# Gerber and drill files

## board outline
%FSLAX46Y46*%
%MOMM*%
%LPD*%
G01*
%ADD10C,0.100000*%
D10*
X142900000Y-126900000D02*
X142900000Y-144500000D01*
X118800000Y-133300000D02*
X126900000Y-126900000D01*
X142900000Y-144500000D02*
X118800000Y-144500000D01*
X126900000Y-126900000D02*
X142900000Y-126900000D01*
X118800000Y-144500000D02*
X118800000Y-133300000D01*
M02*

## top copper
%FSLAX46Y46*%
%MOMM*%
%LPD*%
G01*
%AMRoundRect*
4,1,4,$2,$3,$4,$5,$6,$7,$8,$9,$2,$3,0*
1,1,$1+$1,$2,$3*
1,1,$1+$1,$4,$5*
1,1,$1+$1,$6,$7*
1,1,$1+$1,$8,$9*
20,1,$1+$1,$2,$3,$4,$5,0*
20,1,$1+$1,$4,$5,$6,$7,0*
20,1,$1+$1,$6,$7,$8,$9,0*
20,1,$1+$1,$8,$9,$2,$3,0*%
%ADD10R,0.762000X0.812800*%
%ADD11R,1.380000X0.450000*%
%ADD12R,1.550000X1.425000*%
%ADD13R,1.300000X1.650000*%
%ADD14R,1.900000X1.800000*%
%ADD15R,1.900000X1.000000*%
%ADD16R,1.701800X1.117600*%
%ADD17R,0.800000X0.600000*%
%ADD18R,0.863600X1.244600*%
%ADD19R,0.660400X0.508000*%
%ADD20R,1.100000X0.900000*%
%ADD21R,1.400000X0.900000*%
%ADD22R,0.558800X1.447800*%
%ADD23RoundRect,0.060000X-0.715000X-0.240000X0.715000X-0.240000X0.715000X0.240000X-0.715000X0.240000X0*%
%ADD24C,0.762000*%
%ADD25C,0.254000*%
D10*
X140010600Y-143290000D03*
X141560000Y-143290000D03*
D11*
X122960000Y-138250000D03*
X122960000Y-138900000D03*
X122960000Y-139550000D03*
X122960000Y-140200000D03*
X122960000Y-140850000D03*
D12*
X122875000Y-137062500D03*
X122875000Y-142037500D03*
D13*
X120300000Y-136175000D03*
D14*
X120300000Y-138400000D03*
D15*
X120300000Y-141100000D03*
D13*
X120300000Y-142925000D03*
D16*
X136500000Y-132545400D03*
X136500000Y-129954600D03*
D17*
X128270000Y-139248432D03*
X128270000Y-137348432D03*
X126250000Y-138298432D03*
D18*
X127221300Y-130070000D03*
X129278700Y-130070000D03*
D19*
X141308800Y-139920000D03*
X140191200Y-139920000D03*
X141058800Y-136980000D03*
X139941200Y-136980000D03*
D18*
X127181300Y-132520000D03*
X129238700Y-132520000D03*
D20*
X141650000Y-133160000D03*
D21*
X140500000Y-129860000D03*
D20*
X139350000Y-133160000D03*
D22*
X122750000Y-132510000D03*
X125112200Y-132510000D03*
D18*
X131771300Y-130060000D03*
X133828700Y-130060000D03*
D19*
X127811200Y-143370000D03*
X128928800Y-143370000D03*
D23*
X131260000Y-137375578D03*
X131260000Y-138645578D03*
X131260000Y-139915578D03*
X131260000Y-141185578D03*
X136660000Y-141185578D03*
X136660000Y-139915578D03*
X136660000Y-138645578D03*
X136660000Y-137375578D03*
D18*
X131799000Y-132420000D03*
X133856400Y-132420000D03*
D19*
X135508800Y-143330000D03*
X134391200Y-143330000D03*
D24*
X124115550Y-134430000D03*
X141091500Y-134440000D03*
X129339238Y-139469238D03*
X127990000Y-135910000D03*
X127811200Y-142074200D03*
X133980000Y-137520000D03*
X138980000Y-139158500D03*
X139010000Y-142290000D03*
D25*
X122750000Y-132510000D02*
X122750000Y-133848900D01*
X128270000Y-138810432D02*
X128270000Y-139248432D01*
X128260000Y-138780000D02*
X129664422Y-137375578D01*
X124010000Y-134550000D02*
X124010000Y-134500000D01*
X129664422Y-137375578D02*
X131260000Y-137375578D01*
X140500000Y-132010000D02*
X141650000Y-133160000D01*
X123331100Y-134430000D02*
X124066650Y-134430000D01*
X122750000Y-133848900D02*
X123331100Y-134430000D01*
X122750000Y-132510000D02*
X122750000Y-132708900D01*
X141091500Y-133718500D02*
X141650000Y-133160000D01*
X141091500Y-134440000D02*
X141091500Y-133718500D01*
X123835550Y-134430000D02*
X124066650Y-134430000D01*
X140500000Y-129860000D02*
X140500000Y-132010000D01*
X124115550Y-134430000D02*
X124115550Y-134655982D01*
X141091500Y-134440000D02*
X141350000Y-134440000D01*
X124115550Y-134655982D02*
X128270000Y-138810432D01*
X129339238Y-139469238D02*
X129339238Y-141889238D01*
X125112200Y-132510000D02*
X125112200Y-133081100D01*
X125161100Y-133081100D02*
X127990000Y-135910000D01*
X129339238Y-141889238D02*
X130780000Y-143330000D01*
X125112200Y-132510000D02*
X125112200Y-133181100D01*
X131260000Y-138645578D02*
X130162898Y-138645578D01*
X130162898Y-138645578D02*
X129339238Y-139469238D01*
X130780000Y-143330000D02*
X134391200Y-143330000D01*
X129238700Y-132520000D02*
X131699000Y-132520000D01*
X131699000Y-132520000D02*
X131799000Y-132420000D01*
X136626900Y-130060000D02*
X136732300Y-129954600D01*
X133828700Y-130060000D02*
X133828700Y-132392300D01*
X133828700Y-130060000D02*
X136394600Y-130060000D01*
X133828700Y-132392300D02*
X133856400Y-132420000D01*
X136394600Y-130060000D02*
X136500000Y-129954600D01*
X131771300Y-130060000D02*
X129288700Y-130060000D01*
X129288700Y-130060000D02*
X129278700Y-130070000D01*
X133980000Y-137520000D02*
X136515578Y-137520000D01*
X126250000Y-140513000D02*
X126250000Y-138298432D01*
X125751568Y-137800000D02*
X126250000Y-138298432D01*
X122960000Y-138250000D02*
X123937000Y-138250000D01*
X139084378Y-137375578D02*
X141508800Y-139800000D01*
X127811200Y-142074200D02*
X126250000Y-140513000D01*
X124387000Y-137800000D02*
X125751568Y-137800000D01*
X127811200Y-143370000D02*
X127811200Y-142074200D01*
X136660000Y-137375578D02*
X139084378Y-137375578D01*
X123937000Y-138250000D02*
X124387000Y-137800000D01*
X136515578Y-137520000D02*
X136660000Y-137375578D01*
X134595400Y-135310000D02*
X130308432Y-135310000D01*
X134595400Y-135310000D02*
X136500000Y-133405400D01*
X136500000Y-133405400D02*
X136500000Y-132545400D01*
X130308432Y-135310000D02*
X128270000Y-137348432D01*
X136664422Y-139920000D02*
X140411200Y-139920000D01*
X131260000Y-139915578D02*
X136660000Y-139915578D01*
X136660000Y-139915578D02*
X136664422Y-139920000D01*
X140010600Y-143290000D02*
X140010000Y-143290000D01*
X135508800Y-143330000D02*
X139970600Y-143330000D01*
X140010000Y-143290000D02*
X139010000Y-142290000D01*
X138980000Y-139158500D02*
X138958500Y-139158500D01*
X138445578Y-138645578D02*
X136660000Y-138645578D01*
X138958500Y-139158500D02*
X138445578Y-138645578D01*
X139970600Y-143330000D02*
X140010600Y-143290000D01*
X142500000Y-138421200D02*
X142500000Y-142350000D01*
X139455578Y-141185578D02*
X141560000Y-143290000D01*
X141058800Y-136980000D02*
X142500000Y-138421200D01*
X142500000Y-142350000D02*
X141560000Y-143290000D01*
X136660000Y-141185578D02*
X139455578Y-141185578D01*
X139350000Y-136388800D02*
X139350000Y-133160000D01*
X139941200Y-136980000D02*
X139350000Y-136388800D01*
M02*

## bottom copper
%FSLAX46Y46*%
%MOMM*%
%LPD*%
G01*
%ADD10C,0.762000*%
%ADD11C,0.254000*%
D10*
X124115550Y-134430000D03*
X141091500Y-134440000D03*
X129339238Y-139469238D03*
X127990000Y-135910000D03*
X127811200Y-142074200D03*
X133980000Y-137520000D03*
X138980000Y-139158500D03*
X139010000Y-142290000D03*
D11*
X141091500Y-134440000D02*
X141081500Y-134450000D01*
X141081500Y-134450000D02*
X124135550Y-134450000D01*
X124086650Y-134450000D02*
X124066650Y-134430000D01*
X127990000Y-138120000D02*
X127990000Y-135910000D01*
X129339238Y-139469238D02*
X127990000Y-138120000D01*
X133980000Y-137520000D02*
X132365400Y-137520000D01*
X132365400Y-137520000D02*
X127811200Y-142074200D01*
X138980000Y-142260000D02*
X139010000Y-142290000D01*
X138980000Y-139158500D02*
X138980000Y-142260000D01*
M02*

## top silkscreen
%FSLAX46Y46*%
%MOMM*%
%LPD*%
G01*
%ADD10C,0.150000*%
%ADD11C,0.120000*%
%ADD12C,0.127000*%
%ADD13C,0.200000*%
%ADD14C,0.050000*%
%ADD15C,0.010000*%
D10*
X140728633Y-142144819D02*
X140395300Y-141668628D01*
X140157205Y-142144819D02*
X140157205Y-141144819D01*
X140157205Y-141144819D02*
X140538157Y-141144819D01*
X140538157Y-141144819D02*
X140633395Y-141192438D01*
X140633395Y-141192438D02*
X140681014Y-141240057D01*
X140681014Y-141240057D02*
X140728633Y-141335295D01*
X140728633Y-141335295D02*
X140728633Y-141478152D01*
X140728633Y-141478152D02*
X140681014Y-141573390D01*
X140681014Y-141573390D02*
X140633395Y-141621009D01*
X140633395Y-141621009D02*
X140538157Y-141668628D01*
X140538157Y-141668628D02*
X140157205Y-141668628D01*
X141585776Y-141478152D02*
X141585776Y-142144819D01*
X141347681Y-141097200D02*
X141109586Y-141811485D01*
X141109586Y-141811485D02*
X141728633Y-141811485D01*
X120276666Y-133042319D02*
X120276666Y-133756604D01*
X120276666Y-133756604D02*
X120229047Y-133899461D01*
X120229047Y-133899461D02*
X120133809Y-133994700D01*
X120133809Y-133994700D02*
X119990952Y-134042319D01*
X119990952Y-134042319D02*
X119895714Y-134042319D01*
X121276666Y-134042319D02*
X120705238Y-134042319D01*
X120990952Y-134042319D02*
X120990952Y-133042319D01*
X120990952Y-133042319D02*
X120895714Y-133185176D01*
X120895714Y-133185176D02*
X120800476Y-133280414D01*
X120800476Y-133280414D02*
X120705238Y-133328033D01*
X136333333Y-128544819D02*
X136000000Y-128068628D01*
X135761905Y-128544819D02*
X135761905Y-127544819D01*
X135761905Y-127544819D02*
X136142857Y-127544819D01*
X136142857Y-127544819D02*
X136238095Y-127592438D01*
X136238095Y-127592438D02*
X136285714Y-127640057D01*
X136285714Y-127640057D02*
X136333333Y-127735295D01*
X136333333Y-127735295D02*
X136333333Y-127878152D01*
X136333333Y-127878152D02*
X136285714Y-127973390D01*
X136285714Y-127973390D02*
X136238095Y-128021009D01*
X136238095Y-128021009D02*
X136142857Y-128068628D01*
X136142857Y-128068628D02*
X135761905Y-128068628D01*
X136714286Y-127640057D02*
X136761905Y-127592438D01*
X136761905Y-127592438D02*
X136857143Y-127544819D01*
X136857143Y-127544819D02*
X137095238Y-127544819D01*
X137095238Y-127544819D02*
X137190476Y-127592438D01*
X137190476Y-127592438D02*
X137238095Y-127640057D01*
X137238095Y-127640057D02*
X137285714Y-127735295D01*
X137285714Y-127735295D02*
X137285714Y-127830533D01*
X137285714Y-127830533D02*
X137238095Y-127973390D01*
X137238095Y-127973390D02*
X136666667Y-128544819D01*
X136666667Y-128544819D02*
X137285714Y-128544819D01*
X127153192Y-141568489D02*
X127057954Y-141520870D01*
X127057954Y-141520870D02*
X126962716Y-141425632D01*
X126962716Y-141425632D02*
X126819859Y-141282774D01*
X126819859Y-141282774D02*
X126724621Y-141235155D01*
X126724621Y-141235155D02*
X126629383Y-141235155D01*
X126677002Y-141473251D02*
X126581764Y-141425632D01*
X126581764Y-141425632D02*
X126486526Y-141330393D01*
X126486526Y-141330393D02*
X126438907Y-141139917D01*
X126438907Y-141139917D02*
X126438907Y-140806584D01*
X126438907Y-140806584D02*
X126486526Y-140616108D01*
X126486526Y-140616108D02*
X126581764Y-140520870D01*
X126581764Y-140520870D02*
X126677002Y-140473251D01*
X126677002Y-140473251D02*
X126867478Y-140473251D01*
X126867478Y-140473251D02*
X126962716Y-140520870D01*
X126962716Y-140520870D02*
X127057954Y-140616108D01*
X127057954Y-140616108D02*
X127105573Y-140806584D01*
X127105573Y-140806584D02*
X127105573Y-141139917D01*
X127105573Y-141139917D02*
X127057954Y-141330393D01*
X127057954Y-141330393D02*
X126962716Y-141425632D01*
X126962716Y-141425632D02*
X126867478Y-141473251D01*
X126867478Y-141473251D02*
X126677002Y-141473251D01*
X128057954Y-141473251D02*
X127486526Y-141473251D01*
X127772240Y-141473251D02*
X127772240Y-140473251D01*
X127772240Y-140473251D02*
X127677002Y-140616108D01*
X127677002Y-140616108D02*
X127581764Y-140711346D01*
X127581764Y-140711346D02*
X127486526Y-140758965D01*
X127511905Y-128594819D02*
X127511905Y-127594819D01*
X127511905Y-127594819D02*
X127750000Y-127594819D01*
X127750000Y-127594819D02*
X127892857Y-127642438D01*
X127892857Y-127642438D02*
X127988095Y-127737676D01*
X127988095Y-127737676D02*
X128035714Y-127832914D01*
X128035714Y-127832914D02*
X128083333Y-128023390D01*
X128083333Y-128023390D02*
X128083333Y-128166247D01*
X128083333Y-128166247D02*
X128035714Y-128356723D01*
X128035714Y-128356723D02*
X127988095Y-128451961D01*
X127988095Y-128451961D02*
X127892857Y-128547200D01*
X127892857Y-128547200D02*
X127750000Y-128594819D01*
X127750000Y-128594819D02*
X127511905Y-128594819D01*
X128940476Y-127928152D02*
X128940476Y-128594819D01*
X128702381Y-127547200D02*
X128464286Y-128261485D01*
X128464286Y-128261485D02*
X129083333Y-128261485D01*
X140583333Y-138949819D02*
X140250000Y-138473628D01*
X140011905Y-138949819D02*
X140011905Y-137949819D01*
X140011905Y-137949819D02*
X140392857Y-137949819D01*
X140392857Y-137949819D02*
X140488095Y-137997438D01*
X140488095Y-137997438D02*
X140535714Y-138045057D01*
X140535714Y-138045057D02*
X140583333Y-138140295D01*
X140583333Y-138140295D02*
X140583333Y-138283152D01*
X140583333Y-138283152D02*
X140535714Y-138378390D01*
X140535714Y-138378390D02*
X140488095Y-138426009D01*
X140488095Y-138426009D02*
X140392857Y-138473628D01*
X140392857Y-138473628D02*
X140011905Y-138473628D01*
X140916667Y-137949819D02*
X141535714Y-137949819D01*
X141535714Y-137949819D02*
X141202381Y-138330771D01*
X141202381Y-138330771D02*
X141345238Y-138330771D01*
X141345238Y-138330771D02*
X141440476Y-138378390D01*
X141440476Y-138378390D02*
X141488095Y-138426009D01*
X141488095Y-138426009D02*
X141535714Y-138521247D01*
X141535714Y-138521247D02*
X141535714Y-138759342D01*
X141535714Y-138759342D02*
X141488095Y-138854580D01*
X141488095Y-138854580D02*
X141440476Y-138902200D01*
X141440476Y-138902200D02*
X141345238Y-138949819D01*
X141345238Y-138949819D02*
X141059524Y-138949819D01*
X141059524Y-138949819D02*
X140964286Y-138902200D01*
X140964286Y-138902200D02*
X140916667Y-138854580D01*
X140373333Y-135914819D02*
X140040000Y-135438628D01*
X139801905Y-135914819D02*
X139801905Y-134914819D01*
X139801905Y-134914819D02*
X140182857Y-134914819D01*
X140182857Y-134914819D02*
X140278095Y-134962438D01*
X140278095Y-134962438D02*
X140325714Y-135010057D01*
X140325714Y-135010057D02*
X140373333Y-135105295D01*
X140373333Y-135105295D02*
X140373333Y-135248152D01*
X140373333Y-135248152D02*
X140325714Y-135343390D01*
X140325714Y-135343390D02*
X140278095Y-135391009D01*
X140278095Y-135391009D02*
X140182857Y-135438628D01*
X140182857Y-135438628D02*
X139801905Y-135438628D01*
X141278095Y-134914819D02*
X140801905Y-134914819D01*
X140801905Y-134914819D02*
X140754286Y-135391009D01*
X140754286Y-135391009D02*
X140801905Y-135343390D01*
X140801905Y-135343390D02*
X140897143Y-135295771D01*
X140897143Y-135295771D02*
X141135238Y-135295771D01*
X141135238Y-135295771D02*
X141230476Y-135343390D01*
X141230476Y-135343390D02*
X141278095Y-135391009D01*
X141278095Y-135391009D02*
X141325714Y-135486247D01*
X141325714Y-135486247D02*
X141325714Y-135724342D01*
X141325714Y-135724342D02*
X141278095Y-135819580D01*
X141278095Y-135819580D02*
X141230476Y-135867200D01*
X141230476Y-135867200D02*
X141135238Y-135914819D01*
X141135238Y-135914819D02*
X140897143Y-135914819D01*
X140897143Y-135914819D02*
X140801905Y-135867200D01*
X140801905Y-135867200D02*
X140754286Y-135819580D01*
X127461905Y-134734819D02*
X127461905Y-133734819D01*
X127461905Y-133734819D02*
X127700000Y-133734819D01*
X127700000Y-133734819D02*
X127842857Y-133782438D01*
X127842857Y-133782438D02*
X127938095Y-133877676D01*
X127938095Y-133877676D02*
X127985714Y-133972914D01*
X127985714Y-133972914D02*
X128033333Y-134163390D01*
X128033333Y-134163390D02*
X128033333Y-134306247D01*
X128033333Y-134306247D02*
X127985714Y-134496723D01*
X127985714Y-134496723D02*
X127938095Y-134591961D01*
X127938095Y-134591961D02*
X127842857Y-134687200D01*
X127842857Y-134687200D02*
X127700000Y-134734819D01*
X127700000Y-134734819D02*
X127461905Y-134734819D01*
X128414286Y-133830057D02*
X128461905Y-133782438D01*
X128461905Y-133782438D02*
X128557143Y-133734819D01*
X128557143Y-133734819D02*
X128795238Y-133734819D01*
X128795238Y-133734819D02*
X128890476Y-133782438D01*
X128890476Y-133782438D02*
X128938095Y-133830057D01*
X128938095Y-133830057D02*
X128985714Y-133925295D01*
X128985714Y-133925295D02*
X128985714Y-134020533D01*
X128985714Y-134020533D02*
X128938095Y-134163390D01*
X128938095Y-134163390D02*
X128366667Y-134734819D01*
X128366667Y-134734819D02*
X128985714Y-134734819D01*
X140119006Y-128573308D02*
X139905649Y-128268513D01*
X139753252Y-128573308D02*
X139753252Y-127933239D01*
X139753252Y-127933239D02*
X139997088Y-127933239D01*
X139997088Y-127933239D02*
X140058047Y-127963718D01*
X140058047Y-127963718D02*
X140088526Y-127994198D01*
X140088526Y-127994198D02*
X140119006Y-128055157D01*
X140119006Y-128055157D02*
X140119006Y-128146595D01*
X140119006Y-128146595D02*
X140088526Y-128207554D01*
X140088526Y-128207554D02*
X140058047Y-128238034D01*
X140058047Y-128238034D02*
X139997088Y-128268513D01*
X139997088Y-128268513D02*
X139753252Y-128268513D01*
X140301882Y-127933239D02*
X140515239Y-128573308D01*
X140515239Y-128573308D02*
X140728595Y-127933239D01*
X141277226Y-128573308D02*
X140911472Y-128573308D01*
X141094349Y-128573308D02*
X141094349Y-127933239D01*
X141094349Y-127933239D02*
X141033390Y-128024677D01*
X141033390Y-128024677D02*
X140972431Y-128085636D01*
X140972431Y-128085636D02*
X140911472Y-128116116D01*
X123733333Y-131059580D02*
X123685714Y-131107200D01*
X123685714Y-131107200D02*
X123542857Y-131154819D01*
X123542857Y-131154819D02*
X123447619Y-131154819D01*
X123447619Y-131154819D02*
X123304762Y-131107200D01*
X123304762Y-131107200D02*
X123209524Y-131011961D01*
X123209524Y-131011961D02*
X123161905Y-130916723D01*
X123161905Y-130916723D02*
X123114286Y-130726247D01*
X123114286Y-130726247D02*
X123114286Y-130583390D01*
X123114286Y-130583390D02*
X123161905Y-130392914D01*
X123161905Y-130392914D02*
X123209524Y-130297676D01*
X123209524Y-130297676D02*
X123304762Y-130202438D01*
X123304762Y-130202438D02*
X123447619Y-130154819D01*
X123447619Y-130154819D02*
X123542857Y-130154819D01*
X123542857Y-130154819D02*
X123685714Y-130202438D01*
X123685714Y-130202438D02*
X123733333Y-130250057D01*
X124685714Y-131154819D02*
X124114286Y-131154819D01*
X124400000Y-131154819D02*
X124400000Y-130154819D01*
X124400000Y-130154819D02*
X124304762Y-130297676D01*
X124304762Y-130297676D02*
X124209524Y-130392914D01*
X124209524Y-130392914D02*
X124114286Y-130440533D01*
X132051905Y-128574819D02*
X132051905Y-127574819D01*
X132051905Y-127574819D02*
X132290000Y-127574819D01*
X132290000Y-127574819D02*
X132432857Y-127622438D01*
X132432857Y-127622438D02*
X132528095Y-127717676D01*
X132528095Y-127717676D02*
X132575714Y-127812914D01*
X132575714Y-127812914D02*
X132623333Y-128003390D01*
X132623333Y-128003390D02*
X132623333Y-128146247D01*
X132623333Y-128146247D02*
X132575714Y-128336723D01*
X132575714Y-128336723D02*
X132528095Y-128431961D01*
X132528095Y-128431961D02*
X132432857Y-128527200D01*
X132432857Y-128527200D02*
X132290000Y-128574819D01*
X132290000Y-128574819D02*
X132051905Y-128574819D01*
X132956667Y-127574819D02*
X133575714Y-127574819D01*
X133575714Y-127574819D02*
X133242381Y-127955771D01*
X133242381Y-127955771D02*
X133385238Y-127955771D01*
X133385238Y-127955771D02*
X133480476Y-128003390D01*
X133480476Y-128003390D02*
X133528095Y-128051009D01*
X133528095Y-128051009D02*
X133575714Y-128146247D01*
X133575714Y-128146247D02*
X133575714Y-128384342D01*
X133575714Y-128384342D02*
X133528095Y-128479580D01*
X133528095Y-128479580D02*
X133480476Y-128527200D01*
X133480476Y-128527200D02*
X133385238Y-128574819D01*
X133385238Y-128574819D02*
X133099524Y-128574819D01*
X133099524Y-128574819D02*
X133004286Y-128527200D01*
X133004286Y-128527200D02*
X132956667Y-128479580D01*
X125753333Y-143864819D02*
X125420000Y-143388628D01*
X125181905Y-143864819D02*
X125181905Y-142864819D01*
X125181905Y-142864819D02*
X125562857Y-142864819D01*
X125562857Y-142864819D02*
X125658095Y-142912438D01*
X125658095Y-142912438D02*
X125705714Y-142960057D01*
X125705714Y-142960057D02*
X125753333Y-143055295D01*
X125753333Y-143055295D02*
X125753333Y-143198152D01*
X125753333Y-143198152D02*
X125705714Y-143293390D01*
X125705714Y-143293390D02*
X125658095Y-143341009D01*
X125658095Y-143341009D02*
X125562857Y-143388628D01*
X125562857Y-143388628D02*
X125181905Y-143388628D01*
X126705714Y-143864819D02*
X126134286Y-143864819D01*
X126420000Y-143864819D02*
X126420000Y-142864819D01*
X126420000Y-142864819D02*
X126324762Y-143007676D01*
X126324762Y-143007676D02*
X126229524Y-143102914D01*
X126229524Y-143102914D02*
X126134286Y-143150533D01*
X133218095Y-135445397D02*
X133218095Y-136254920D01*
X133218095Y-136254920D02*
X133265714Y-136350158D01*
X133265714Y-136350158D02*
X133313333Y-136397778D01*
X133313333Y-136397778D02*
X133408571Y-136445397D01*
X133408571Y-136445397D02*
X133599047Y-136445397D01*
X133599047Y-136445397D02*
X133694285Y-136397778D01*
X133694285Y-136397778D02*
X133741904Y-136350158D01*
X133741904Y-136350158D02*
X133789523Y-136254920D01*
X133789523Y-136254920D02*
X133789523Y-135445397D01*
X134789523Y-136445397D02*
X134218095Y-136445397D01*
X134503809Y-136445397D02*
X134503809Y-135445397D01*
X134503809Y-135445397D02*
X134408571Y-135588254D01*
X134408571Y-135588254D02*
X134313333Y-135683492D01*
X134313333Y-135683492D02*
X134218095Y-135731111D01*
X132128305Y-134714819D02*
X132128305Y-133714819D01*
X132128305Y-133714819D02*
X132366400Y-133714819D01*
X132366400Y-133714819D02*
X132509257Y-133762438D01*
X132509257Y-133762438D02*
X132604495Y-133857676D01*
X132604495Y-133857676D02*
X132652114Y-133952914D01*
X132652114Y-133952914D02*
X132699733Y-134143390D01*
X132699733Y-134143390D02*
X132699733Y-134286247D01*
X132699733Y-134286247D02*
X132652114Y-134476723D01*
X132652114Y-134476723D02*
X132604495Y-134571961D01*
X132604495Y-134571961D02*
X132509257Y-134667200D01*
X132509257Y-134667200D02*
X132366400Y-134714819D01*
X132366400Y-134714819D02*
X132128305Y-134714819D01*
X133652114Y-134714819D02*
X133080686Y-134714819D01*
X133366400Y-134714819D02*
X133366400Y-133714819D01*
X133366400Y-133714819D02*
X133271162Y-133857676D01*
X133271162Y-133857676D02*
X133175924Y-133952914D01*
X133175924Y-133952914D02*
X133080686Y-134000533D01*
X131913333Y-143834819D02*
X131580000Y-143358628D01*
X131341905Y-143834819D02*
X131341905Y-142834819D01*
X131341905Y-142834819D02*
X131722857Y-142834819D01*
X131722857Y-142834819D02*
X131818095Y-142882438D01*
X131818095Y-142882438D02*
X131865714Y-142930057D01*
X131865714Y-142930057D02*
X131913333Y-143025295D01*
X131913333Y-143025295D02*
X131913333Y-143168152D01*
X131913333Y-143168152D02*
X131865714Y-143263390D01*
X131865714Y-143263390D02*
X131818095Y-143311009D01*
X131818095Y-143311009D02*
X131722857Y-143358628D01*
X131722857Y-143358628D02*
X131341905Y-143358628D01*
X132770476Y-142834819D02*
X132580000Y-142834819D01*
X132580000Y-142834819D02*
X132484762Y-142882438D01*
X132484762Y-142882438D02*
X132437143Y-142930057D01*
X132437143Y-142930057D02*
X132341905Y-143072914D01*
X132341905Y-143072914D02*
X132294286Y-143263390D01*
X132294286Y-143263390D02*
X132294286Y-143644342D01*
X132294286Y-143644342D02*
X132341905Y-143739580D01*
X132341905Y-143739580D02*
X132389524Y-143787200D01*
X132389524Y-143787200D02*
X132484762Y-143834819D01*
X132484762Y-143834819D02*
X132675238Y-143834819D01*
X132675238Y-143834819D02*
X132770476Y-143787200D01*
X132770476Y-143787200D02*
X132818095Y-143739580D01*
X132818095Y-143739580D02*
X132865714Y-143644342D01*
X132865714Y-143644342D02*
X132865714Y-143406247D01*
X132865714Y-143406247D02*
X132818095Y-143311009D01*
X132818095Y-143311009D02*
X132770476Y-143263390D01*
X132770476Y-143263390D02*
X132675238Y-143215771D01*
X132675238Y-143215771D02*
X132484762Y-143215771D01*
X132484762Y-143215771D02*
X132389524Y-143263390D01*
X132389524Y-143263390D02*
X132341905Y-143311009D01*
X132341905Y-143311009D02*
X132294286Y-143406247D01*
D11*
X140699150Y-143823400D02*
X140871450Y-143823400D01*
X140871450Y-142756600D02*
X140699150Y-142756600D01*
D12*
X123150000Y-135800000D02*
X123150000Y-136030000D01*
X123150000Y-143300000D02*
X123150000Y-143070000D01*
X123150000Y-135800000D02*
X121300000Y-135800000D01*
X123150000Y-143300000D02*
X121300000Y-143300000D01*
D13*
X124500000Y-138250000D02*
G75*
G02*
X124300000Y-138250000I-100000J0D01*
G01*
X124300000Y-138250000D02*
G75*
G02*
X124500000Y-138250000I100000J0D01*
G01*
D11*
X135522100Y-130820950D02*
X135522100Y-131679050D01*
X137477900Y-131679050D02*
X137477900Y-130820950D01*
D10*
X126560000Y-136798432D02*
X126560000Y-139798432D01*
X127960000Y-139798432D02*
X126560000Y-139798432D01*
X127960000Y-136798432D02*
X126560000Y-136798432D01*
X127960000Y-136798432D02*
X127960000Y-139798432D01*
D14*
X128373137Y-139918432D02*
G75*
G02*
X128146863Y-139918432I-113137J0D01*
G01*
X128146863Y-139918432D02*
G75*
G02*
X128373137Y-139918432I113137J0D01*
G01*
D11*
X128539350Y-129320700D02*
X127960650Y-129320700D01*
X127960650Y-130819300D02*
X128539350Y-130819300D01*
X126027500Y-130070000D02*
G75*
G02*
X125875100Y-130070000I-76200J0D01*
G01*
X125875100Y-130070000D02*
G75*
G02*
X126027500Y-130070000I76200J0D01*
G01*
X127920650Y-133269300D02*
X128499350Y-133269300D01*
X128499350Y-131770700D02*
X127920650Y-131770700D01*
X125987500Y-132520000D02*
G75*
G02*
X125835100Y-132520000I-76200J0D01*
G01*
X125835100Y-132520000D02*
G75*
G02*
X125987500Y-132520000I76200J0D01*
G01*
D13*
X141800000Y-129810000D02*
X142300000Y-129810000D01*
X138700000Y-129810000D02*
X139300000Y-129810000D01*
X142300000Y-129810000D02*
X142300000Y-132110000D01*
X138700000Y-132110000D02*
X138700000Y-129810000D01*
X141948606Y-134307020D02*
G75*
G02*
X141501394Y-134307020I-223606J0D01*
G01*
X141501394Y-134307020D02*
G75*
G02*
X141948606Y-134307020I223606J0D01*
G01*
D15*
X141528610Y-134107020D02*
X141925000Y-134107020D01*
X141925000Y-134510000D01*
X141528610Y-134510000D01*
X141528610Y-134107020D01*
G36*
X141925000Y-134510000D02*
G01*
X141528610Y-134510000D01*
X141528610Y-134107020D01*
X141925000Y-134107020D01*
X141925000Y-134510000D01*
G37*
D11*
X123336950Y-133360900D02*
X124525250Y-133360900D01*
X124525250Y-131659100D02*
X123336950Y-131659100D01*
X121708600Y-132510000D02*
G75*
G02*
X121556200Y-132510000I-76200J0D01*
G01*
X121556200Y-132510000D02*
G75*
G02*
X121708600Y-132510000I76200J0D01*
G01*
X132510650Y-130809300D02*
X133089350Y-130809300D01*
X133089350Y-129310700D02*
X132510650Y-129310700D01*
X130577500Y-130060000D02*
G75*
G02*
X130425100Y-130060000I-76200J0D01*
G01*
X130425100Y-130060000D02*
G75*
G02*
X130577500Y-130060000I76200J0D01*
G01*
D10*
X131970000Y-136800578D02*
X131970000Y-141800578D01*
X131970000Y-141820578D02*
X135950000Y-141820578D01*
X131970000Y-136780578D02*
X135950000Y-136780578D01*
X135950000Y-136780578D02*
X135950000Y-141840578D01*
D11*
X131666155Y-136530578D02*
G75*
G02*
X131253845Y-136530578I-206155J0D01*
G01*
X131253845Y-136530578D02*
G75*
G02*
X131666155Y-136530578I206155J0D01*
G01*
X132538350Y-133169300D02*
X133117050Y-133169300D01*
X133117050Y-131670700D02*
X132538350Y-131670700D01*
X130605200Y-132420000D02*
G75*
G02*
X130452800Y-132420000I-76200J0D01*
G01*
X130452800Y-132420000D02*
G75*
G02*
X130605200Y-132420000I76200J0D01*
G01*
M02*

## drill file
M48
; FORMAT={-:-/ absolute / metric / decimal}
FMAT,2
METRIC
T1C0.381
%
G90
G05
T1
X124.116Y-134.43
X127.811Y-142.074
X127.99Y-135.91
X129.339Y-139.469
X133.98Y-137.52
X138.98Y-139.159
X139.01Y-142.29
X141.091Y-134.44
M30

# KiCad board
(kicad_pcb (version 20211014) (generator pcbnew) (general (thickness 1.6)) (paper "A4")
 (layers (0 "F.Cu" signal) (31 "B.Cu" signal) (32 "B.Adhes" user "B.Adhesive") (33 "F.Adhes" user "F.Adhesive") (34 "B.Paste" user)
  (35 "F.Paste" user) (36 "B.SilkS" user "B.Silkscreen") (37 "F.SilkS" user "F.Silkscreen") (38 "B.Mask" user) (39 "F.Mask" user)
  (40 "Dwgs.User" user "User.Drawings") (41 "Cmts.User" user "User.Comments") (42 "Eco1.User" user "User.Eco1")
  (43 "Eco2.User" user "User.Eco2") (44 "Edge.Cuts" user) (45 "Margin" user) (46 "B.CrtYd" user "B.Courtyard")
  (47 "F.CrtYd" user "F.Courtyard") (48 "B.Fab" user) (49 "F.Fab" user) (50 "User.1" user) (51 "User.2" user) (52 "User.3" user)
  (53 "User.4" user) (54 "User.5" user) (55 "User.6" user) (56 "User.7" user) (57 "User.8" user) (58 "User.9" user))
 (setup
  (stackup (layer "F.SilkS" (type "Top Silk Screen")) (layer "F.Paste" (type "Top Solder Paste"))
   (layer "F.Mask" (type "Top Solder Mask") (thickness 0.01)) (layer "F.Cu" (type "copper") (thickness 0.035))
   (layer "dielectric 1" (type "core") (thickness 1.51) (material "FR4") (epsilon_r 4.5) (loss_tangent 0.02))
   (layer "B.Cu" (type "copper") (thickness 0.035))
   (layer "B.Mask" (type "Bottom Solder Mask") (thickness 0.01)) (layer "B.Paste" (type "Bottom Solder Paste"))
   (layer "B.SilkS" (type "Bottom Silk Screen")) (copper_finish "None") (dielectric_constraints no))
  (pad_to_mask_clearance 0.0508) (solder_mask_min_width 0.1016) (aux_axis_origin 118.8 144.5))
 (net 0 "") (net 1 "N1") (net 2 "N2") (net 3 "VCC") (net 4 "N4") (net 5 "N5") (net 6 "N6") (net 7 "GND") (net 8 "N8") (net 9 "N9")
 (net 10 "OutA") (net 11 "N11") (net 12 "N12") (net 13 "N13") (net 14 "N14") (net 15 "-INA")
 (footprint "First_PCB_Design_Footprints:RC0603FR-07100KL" (layer "F.Cu") (at 140.7853 143.29)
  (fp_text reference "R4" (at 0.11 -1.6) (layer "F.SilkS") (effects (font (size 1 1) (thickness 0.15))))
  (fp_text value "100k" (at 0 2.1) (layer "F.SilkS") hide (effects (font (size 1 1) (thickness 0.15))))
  (fp_line (start -0.08615 0.5334) (end 0.08615 0.5334) (layer "F.SilkS") (width 0.12))
  (fp_line (start 0.08615 -0.5334) (end -0.08615 -0.5334) (layer "F.SilkS") (width 0.12))
  (pad "1" smd rect (at -0.7747 0) (size 0.762 0.8128) (layers "F.Cu" "F.Paste" "F.Mask") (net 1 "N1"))
  (pad "2" smd rect (at 0.7747 0) (size 0.762 0.8128) (layers "F.Cu" "F.Paste" "F.Mask") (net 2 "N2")))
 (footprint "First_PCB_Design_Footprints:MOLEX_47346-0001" (layer "F.Cu") (at 120.3 139.55 -90)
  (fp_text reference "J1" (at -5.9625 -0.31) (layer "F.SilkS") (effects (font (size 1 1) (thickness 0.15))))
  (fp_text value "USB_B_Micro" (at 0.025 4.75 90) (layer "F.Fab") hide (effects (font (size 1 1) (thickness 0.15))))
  (fp_line (start -3.75 -2.85) (end -3.52 -2.85) (layer "F.SilkS") (width 0.127))
  (fp_line (start 3.75 -2.85) (end 3.52 -2.85) (layer "F.SilkS") (width 0.127))
  (fp_line (start -3.75 -2.85) (end -3.75 -1) (layer "F.SilkS") (width 0.127))
  (fp_line (start 3.75 -2.85) (end 3.75 -1) (layer "F.SilkS") (width 0.127))
  (fp_circle (center -1.3 -4.1) (end -1.2 -4.1) (layer "F.SilkS") (width 0.2) (fill none))
  (pad "1" smd rect (at -1.3 -2.66 270) (size 0.45 1.38) (layers "F.Cu" "F.Paste" "F.Mask") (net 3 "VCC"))
  (pad "2" smd rect (at -0.65 -2.66 270) (size 0.45 1.38) (layers "F.Cu" "F.Paste" "F.Mask") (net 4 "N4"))
  (pad "3" smd rect (at 0 -2.66 270) (size 0.45 1.38) (layers "F.Cu" "F.Paste" "F.Mask") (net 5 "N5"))
  (pad "4" smd rect (at 0.65 -2.66 270) (size 0.45 1.38) (layers "F.Cu" "F.Paste" "F.Mask") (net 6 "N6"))
  (pad "5" smd rect (at 1.3 -2.66 270) (size 0.45 1.38) (layers "F.Cu" "F.Paste" "F.Mask") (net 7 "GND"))
  (pad "S1" smd rect (at -2.4875 -2.575 270) (size 1.425 1.55) (layers "F.Cu" "F.Paste" "F.Mask"))
  (pad "S2" smd rect (at 2.4875 -2.575 270) (size 1.425 1.55) (layers "F.Cu" "F.Paste" "F.Mask"))
  (pad "S3" smd rect (at -3.375 0 270) (size 1.65 1.3) (layers "F.Cu" "F.Paste" "F.Mask"))
  (pad "S4" smd rect (at -1.15 0 270) (size 1.8 1.9) (layers "F.Cu" "F.Paste" "F.Mask"))
  (pad "S5" smd rect (at 1.55 0 270) (size 1 1.9) (layers "F.Cu" "F.Paste" "F.Mask"))
  (pad "S6" smd rect (at 3.375 0 270) (size 1.65 1.3) (layers "F.Cu" "F.Paste" "F.Mask")))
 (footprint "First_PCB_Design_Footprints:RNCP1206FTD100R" (layer "F.Cu") (at 136.5 131.25 90)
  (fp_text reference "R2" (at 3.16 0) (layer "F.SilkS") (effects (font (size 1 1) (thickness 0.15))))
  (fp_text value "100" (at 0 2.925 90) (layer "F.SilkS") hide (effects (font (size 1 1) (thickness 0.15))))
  (fp_line (start 0.42905 -0.9779) (end -0.42905 -0.9779) (layer "F.SilkS") (width 0.12))
  (fp_line (start -0.42905 0.9779) (end 0.42905 0.9779) (layer "F.SilkS") (width 0.12))
  (pad "1" smd rect (at -1.2954 0 90) (size 1.1176 1.7018) (layers "F.Cu" "F.Paste" "F.Mask") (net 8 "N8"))
  (pad "2" smd rect (at 1.2954 0 90) (size 1.1176 1.7018) (layers "F.Cu" "F.Paste" "F.Mask") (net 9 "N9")))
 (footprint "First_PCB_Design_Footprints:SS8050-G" (layer "F.Cu") (at 127.26 138.298432 90)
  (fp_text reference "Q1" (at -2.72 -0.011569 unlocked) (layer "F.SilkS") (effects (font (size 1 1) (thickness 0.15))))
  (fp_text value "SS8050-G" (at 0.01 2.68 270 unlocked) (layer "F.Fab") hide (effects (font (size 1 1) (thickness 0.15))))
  (fp_line (start 1.5 -0.7) (end -1.5 -0.7) (layer "F.SilkS") (width 0.15))
  (fp_line (start -1.5 0.7) (end -1.5 -0.7) (layer "F.SilkS") (width 0.15))
  (fp_line (start 1.5 0.7) (end 1.5 -0.7) (layer "F.SilkS") (width 0.15))
  (fp_line (start 1.5 0.7) (end -1.5 0.7) (layer "F.SilkS") (width 0.15))
  (fp_circle (center -1.62 1) (end -1.506863 1) (layer "F.SilkS") (width 0.05) (fill none))
  (pad "1" smd rect (at -0.95 1.01 90) (size 0.6 0.8) (layers *.Mask "F.Cu") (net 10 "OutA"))
  (pad "2" smd rect (at 0.95 1.01 90) (size 0.6 0.8) (layers *.Mask "F.Cu") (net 8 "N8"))
  (pad "3" smd rect (at 0 -1.01 90) (size 0.6 0.8) (layers *.Mask "F.Cu") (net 3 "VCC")))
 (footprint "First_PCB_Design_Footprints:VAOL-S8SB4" (layer "F.Cu") (at 128.25 130.07)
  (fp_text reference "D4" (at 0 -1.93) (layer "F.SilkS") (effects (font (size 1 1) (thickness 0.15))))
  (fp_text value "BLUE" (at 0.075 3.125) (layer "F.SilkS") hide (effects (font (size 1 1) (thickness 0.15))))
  (fp_line (start 0.28935 -0.7493) (end -0.28935 -0.7493) (layer "F.SilkS") (width 0.12))
  (fp_line (start -0.28935 0.7493) (end 0.28935 0.7493) (layer "F.SilkS") (width 0.12))
  (fp_circle (center -2.2987 0) (end -2.2225 0) (layer "F.SilkS") (width 0.12) (fill none))
  (pad "1" smd rect (at -1.0287 0) (size 0.8636 1.2446) (layers "F.Cu" "F.Paste" "F.Mask") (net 7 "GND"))
  (pad "2" smd rect (at 1.0287 0) (size 0.8636 1.2446) (layers "F.Cu" "F.Paste" "F.Mask") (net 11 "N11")))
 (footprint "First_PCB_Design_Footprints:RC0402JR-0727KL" (layer "F.Cu") (at 140.75 139.92 180)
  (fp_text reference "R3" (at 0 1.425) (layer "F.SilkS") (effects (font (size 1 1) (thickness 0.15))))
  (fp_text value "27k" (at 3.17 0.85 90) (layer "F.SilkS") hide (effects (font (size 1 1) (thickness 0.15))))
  (pad "1" smd rect (at -0.5588 0 180) (size 0.6604 0.508) (layers "F.Cu" "F.Paste" "F.Mask") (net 3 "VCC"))
  (pad "2" smd rect (at 0.5588 0 180) (size 0.6604 0.508) (layers "F.Cu" "F.Paste" "F.Mask") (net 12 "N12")))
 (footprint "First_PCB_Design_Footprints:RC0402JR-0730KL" (layer "F.Cu") (at 140.5 136.98 180)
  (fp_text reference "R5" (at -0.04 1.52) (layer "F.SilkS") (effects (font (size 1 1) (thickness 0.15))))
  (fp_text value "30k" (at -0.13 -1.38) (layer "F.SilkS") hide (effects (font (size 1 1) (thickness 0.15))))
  (pad "1" smd rect (at -0.5588 0 180) (size 0.6604 0.508) (layers "F.Cu" "F.Paste" "F.Mask") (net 2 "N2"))
  (pad "2" smd rect (at 0.5588 0 180) (size 0.6604 0.508) (layers "F.Cu" "F.Paste" "F.Mask") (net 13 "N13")))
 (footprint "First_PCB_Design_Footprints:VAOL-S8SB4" (layer "F.Cu") (at 128.21 132.52)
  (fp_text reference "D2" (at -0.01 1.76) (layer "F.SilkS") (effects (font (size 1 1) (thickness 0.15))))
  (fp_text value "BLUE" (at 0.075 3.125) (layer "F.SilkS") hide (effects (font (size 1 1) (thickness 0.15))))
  (fp_line (start -0.28935 0.7493) (end 0.28935 0.7493) (layer "F.SilkS") (width 0.12))
  (fp_line (start 0.28935 -0.7493) (end -0.28935 -0.7493) (layer "F.SilkS") (width 0.12))
  (fp_circle (center -2.2987 0) (end -2.2225 0) (layer "F.SilkS") (width 0.12) (fill none))
  (pad "1" smd rect (at -1.0287 0) (size 0.8636 1.2446) (layers "F.Cu" "F.Paste" "F.Mask") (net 7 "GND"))
  (pad "2" smd rect (at 1.0287 0) (size 0.8636 1.2446) (layers "F.Cu" "F.Paste" "F.Mask") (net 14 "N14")))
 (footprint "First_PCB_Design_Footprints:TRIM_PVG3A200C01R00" (layer "F.Cu") (at 140.5 131.51)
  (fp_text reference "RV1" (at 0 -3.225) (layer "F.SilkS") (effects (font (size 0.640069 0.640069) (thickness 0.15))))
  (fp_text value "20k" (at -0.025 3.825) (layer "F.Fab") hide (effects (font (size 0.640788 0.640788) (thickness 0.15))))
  (fp_line (start 1.3 -1.7) (end 1.8 -1.7) (layer "F.SilkS") (width 0.2))
  (fp_line (start -1.8 -1.7) (end -1.2 -1.7) (layer "F.SilkS") (width 0.2))
  (fp_line (start 1.8 -1.7) (end 1.8 0.6) (layer "F.SilkS") (width 0.2))
  (fp_line (start -1.8 0.6) (end -1.8 -1.7) (layer "F.SilkS") (width 0.2))
  (fp_circle (center 1.225 2.79702) (end 1.448606 2.79702) (layer "F.SilkS") (width 0.2) (fill none))
  (fp_poly (pts (xy 1.02861 2.59702) (xy 1.425 2.59702) (xy 1.425 3) (xy 1.02861 3)) (layer "F.SilkS") (width 0.01) (fill solid))
  (pad "1" smd rect (at 1.15 1.65) (size 1.1 0.9) (layers "F.Cu" "F.Paste" "F.Mask") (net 10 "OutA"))
  (pad "2" smd rect (at 0 -1.65) (size 1.4 0.9) (layers "F.Cu" "F.Paste" "F.Mask") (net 10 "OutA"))
  (pad "3" smd rect (at -1.15 1.65) (size 1.1 0.9) (layers "F.Cu" "F.Paste" "F.Mask") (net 13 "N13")))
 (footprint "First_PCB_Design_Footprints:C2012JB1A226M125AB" (layer "F.Cu") (at 123.9311 132.51)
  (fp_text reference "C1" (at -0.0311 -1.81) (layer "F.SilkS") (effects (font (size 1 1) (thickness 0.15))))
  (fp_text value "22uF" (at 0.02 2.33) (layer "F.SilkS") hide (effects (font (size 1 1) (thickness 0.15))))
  (fp_line (start -0.59415 0.8509) (end 0.59415 0.8509) (layer "F.SilkS") (width 0.12))
  (fp_line (start 0.59415 -0.8509) (end -0.59415 -0.8509) (layer "F.SilkS") (width 0.12))
  (fp_circle (center -2.2987 0) (end -2.2225 0) (layer "F.SilkS") (width 0.12) (fill none))
  (pad "1" smd rect (at -1.1811 0) (size 0.5588 1.4478) (layers "F.Cu" "F.Paste" "F.Mask") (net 10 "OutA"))
  (pad "2" smd rect (at 1.1811 0) (size 0.5588 1.4478) (layers "F.Cu" "F.Paste" "F.Mask") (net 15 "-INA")))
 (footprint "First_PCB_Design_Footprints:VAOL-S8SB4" (layer "F.Cu") (at 132.8 130.06)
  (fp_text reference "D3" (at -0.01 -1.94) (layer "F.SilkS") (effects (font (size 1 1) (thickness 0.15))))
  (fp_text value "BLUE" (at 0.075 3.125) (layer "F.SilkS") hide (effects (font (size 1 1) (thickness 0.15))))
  (fp_line (start -0.28935 0.7493) (end 0.28935 0.7493) (layer "F.SilkS") (width 0.12))
  (fp_line (start 0.28935 -0.7493) (end -0.28935 -0.7493) (layer "F.SilkS") (width 0.12))
  (fp_circle (center -2.2987 0) (end -2.2225 0) (layer "F.SilkS") (width 0.12) (fill none))
  (pad "1" smd rect (at -1.0287 0) (size 0.8636 1.2446) (layers "F.Cu" "F.Paste" "F.Mask") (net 11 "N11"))
  (pad "2" smd rect (at 1.0287 0) (size 0.8636 1.2446) (layers "F.Cu" "F.Paste" "F.Mask") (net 9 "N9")))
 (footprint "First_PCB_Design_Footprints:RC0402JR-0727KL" (layer "F.Cu") (at 128.37 143.37)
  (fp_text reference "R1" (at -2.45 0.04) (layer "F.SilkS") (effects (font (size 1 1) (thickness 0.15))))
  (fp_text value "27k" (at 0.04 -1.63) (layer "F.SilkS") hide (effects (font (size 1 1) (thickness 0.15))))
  (pad "1" smd rect (at -0.5588 0) (size 0.6604 0.508) (layers "F.Cu" "F.Paste" "F.Mask") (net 3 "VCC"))
  (pad "2" smd rect (at 0.5588 0) (size 0.6604 0.508) (layers "F.Cu" "F.Paste" "F.Mask") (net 7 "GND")))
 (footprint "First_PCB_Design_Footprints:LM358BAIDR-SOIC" (layer "F.Cu") (at 133.96 139.280578)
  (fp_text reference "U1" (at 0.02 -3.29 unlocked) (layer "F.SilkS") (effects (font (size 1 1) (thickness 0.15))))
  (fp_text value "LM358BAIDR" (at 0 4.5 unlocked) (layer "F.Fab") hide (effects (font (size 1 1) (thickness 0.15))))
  (fp_line (start -1.99 -2.48) (end -1.99 2.52) (layer "F.SilkS") (width 0.15))
  (fp_line (start -1.99 2.54) (end 1.99 2.54) (layer "F.SilkS") (width 0.15))
  (fp_line (start -1.99 -2.5) (end 1.99 -2.5) (layer "F.SilkS") (width 0.15))
  (fp_line (start 1.99 -2.5) (end 1.99 2.56) (layer "F.SilkS") (width 0.15))
  (fp_circle (center -2.5 -2.75) (end -2.3 -2.7) (layer "F.SilkS") (width 0.12) (fill none))
  (pad "1" smd roundrect (at -2.7 -1.905) (size 1.55 0.6) (layers *.Mask "F.Cu") (roundrect_rratio 0.1) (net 10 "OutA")
   (solder_mask_margin 0.07))
  (pad "2" smd roundrect (at -2.7 -0.635) (size 1.55 0.6) (layers *.Mask "F.Cu") (roundrect_rratio 0.1) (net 15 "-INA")
   (solder_mask_margin 0.07))
  (pad "3" smd roundrect (at -2.7 0.635) (size 1.55 0.6) (layers *.Mask "F.Cu") (roundrect_rratio 0.1) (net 12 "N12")
   (solder_mask_margin 0.07))
  (pad "4" smd roundrect (at -2.7 1.905) (size 1.55 0.6) (layers *.Mask "F.Cu") (roundrect_rratio 0.1) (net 7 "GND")
   (solder_mask_margin 0.07))
  (pad "5" smd roundrect (at 2.7 1.905) (size 1.55 0.6) (layers *.Mask "F.Cu") (roundrect_rratio 0.1) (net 2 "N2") (solder_mask_margin 0.07))
  (pad "6" smd roundrect (at 2.7 0.635) (size 1.55 0.6) (layers *.Mask "F.Cu") (roundrect_rratio 0.1) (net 12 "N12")
   (solder_mask_margin 0.07))
  (pad "7" smd roundrect (at 2.7 -0.635) (size 1.55 0.6) (layers *.Mask "F.Cu") (roundrect_rratio 0.1) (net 1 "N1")
   (solder_mask_margin 0.07))
  (pad "8" smd roundrect (at 2.7 -1.905) (size 1.55 0.6) (layers *.Mask "F.Cu") (roundrect_rratio 0.1) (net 3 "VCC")
   (solder_mask_margin 0.07)))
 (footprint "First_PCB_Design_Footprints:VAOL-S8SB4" (layer "F.Cu") (at 132.8277 132.42)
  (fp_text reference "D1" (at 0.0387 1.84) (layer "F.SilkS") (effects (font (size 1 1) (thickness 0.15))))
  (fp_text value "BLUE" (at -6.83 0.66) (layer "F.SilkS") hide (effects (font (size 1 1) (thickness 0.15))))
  (fp_line (start -0.28935 0.7493) (end 0.28935 0.7493) (layer "F.SilkS") (width 0.12))
  (fp_line (start 0.28935 -0.7493) (end -0.28935 -0.7493) (layer "F.SilkS") (width 0.12))
  (fp_circle (center -2.2987 0) (end -2.2225 0) (layer "F.SilkS") (width 0.12) (fill none))
  (pad "1" smd rect (at -1.0287 0) (size 0.8636 1.2446) (layers "F.Cu" "F.Paste" "F.Mask") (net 14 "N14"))
  (pad "2" smd rect (at 1.0287 0) (size 0.8636 1.2446) (layers "F.Cu" "F.Paste" "F.Mask") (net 9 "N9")))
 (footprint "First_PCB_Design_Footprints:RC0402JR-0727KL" (layer "F.Cu") (at 134.95 143.33 180)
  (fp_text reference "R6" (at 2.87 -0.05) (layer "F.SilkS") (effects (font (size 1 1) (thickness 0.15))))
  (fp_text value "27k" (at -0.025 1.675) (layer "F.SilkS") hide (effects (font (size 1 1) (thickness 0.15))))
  (pad "1" smd rect (at -0.5588 0 180) (size 0.6604 0.508) (layers "F.Cu" "F.Paste" "F.Mask") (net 1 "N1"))
  (pad "2" smd rect (at 0.5588 0 180) (size 0.6604 0.508) (layers "F.Cu" "F.Paste" "F.Mask") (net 15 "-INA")))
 (gr_line (start 142.9 126.9) (end 142.9 144.5) (layer "Edge.Cuts") (width 0.1))
 (gr_line (start 118.8 133.3) (end 126.9 126.9) (layer "Edge.Cuts") (width 0.1))
 (gr_line (start 142.9 144.5) (end 118.8 144.5) (layer "Edge.Cuts") (width 0.1))
 (gr_line (start 126.9 126.9) (end 142.9 126.9) (layer "Edge.Cuts") (width 0.1))
 (gr_line (start 118.8 144.5) (end 118.8 133.3) (layer "Edge.Cuts") (width 0.1))
 (segment (start 122.75 132.51) (end 122.75 133.8489) (width 0.254) (layer "F.Cu") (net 10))
 (segment (start 128.27 138.810432) (end 128.27 139.248432) (width 0.254) (layer "F.Cu") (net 10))
 (segment (start 128.26 138.78) (end 129.664422 137.375578) (width 0.254) (layer "F.Cu") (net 10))
 (segment (start 124.01 134.55) (end 124.01 134.5) (width 0.254) (layer "F.Cu") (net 10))
 (segment (start 129.664422 137.375578) (end 131.26 137.375578) (width 0.254) (layer "F.Cu") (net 10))
 (segment (start 140.5 132.01) (end 141.65 133.16) (width 0.254) (layer "F.Cu") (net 10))
 (segment (start 123.3311 134.43) (end 124.06665 134.43) (width 0.254) (layer "F.Cu") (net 10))
 (segment (start 122.75 133.8489) (end 123.3311 134.43) (width 0.254) (layer "F.Cu") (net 10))
 (segment (start 122.75 132.51) (end 122.75 132.7089) (width 0.254) (layer "F.Cu") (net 10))
 (segment (start 141.0915 133.7185) (end 141.65 133.16) (width 0.254) (layer "F.Cu") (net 10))
 (segment (start 141.0915 134.44) (end 141.0915 133.7185) (width 0.254) (layer "F.Cu") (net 10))
 (segment (start 123.83555 134.43) (end 124.06665 134.43) (width 0.254) (layer "F.Cu") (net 10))
 (segment (start 140.5 129.86) (end 140.5 132.01) (width 0.254) (layer "F.Cu") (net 10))
 (segment (start 124.11555 134.43) (end 124.11555 134.655982) (width 0.254) (layer "F.Cu") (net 10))
 (segment (start 141.0915 134.44) (end 141.35 134.44) (width 0.254) (layer "F.Cu") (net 10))
 (segment (start 124.11555 134.655982) (end 128.27 138.810432) (width 0.254) (layer "F.Cu") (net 10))
 (via (at 124.11555 134.43) (size 0.762) (drill 0.381) (layers "F.Cu" "B.Cu") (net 10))
 (via (at 141.0915 134.44) (size 0.762) (drill 0.381) (layers "F.Cu" "B.Cu") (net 10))
 (segment (start 141.0915 134.44) (end 141.0815 134.45) (width 0.254) (layer "B.Cu") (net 10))
 (segment (start 141.0815 134.45) (end 124.13555 134.45) (width 0.254) (layer "B.Cu") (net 10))
 (segment (start 124.08665 134.45) (end 124.06665 134.43) (width 0.254) (layer "B.Cu") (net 10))
 (segment (start 129.339238 139.469238) (end 129.339238 141.889238) (width 0.254) (layer "F.Cu") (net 15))
 (segment (start 125.1122 132.51) (end 125.1122 133.0811) (width 0.254) (layer "F.Cu") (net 15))
 (segment (start 125.1611 133.0811) (end 127.99 135.91) (width 0.254) (layer "F.Cu") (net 15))
 (segment (start 129.339238 141.889238) (end 130.78 143.33) (width 0.254) (layer "F.Cu") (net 15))
 (segment (start 125.1122 132.51) (end 125.1122 133.1811) (width 0.254) (layer "F.Cu") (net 15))
 (segment (start 131.26 138.645578) (end 130.162898 138.645578) (width 0.254) (layer "F.Cu") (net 15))
 (segment (start 130.162898 138.645578) (end 129.339238 139.469238) (width 0.254) (layer "F.Cu") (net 15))
 (segment (start 130.78 143.33) (end 134.3912 143.33) (width 0.254) (layer "F.Cu") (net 15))
 (via (at 129.339238 139.469238) (size 0.762) (drill 0.381) (layers "F.Cu" "B.Cu") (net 15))
 (via (at 127.99 135.91) (size 0.762) (drill 0.381) (layers "F.Cu" "B.Cu") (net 15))
 (segment (start 127.99 138.12) (end 127.99 135.91) (width 0.254) (layer "B.Cu") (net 15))
 (segment (start 129.339238 139.469238) (end 127.99 138.12) (width 0.254) (layer "B.Cu") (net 15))
 (segment (start 129.2387 132.52) (end 131.699 132.52) (width 0.254) (layer "F.Cu") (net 14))
 (segment (start 131.699 132.52) (end 131.799 132.42) (width 0.254) (layer "F.Cu") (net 14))
 (segment (start 136.6269 130.06) (end 136.7323 129.9546) (width 0.254) (layer "F.Cu") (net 9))
 (segment (start 133.8287 130.06) (end 133.8287 132.3923) (width 0.254) (layer "F.Cu") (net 9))
 (segment (start 133.8287 130.06) (end 136.3946 130.06) (width 0.254) (layer "F.Cu") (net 9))
 (segment (start 133.8287 132.3923) (end 133.8564 132.42) (width 0.254) (layer "F.Cu") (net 9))
 (segment (start 136.3946 130.06) (end 136.5 129.9546) (width 0.254) (layer "F.Cu") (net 9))
 (segment (start 131.7713 130.06) (end 129.2887 130.06) (width 0.254) (layer "F.Cu") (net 11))
 (segment (start 129.2887 130.06) (end 129.2787 130.07) (width 0.254) (layer "F.Cu") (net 11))
 (segment (start 133.98 137.52) (end 136.515578 137.52) (width 0.254) (layer "F.Cu") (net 3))
 (segment (start 126.25 140.513) (end 126.25 138.298432) (width 0.254) (layer "F.Cu") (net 3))
 (segment (start 125.751568 137.8) (end 126.25 138.298432) (width 0.254) (layer "F.Cu") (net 3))
 (segment (start 122.96 138.25) (end 123.937 138.25) (width 0.254) (layer "F.Cu") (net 3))
 (segment (start 139.084378 137.375578) (end 141.5088 139.8) (width 0.254) (layer "F.Cu") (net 3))
 (segment (start 127.8112 142.0742) (end 126.25 140.513) (width 0.254) (layer "F.Cu") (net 3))
 (segment (start 124.387 137.8) (end 125.751568 137.8) (width 0.254) (layer "F.Cu") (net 3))
 (segment (start 127.8112 143.37) (end 127.8112 142.0742) (width 0.254) (layer "F.Cu") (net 3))
 (segment (start 136.66 137.375578) (end 139.084378 137.375578) (width 0.254) (layer "F.Cu") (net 3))
 (segment (start 123.937 138.25) (end 124.387 137.8) (width 0.254) (layer "F.Cu") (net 3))
 (segment (start 136.515578 137.52) (end 136.66 137.375578) (width 0.254) (layer "F.Cu") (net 3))
 (via (at 127.8112 142.0742) (size 0.762) (drill 0.381) (layers "F.Cu" "B.Cu") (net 3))
 (via (at 133.98 137.52) (size 0.762) (drill 0.381) (layers "F.Cu" "B.Cu") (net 3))
 (segment (start 133.98 137.52) (end 132.3654 137.52) (width 0.254) (layer "B.Cu") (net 3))
 (segment (start 132.3654 137.52) (end 127.8112 142.0742) (width 0.254) (layer "B.Cu") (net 3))
 (segment (start 134.5954 135.31) (end 130.308432 135.31) (width 0.254) (layer "F.Cu") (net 8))
 (segment (start 134.5954 135.31) (end 136.5 133.4054) (width 0.254) (layer "F.Cu") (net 8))
 (segment (start 136.5 133.4054) (end 136.5 132.5454) (width 0.254) (layer "F.Cu") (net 8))
 (segment (start 130.308432 135.31) (end 128.27 137.348432) (width 0.254) (layer "F.Cu") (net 8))
 (segment (start 136.664422 139.92) (end 140.4112 139.92) (width 0.254) (layer "F.Cu") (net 12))
 (segment (start 131.26 139.915578) (end 136.66 139.915578) (width 0.254) (layer "F.Cu") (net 12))
 (segment (start 136.66 139.915578) (end 136.664422 139.92) (width 0.254) (layer "F.Cu") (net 12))
 (segment (start 140.0106 143.29) (end 140.01 143.29) (width 0.254) (layer "F.Cu") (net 1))
 (segment (start 135.5088 143.33) (end 139.9706 143.33) (width 0.254) (layer "F.Cu") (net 1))
 (segment (start 140.01 143.29) (end 139.01 142.29) (width 0.254) (layer "F.Cu") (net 1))
 (segment (start 138.98 139.1585) (end 138.9585 139.1585) (width 0.254) (layer "F.Cu") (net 1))
 (segment (start 138.445578 138.645578) (end 136.66 138.645578) (width 0.254) (layer "F.Cu") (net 1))
 (segment (start 138.9585 139.1585) (end 138.445578 138.645578) (width 0.254) (layer "F.Cu") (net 1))
 (segment (start 139.9706 143.33) (end 140.0106 143.29) (width 0.254) (layer "F.Cu") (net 1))
 (via (at 138.98 139.1585) (size 0.762) (drill 0.381) (layers "F.Cu" "B.Cu") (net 1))
 (via (at 139.01 142.29) (size 0.762) (drill 0.381) (layers "F.Cu" "B.Cu") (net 1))
 (segment (start 138.98 142.26) (end 139.01 142.29) (width 0.254) (layer "B.Cu") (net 1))
 (segment (start 138.98 139.1585) (end 138.98 142.26) (width 0.254) (layer "B.Cu") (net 1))
 (segment (start 142.5 138.4212) (end 142.5 142.35) (width 0.254) (layer "F.Cu") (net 2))
 (segment (start 139.455578 141.185578) (end 141.56 143.29) (width 0.254) (layer "F.Cu") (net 2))
 (segment (start 141.0588 136.98) (end 142.5 138.4212) (width 0.254) (layer "F.Cu") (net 2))
 (segment (start 142.5 142.35) (end 141.56 143.29) (width 0.254) (layer "F.Cu") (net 2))
 (segment (start 136.66 141.185578) (end 139.455578 141.185578) (width 0.254) (layer "F.Cu") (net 2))
 (segment (start 139.35 136.3888) (end 139.35 133.16) (width 0.254) (layer "F.Cu") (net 13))
 (segment (start 139.9412 136.98) (end 139.35 136.3888) (width 0.254) (layer "F.Cu") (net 13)))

